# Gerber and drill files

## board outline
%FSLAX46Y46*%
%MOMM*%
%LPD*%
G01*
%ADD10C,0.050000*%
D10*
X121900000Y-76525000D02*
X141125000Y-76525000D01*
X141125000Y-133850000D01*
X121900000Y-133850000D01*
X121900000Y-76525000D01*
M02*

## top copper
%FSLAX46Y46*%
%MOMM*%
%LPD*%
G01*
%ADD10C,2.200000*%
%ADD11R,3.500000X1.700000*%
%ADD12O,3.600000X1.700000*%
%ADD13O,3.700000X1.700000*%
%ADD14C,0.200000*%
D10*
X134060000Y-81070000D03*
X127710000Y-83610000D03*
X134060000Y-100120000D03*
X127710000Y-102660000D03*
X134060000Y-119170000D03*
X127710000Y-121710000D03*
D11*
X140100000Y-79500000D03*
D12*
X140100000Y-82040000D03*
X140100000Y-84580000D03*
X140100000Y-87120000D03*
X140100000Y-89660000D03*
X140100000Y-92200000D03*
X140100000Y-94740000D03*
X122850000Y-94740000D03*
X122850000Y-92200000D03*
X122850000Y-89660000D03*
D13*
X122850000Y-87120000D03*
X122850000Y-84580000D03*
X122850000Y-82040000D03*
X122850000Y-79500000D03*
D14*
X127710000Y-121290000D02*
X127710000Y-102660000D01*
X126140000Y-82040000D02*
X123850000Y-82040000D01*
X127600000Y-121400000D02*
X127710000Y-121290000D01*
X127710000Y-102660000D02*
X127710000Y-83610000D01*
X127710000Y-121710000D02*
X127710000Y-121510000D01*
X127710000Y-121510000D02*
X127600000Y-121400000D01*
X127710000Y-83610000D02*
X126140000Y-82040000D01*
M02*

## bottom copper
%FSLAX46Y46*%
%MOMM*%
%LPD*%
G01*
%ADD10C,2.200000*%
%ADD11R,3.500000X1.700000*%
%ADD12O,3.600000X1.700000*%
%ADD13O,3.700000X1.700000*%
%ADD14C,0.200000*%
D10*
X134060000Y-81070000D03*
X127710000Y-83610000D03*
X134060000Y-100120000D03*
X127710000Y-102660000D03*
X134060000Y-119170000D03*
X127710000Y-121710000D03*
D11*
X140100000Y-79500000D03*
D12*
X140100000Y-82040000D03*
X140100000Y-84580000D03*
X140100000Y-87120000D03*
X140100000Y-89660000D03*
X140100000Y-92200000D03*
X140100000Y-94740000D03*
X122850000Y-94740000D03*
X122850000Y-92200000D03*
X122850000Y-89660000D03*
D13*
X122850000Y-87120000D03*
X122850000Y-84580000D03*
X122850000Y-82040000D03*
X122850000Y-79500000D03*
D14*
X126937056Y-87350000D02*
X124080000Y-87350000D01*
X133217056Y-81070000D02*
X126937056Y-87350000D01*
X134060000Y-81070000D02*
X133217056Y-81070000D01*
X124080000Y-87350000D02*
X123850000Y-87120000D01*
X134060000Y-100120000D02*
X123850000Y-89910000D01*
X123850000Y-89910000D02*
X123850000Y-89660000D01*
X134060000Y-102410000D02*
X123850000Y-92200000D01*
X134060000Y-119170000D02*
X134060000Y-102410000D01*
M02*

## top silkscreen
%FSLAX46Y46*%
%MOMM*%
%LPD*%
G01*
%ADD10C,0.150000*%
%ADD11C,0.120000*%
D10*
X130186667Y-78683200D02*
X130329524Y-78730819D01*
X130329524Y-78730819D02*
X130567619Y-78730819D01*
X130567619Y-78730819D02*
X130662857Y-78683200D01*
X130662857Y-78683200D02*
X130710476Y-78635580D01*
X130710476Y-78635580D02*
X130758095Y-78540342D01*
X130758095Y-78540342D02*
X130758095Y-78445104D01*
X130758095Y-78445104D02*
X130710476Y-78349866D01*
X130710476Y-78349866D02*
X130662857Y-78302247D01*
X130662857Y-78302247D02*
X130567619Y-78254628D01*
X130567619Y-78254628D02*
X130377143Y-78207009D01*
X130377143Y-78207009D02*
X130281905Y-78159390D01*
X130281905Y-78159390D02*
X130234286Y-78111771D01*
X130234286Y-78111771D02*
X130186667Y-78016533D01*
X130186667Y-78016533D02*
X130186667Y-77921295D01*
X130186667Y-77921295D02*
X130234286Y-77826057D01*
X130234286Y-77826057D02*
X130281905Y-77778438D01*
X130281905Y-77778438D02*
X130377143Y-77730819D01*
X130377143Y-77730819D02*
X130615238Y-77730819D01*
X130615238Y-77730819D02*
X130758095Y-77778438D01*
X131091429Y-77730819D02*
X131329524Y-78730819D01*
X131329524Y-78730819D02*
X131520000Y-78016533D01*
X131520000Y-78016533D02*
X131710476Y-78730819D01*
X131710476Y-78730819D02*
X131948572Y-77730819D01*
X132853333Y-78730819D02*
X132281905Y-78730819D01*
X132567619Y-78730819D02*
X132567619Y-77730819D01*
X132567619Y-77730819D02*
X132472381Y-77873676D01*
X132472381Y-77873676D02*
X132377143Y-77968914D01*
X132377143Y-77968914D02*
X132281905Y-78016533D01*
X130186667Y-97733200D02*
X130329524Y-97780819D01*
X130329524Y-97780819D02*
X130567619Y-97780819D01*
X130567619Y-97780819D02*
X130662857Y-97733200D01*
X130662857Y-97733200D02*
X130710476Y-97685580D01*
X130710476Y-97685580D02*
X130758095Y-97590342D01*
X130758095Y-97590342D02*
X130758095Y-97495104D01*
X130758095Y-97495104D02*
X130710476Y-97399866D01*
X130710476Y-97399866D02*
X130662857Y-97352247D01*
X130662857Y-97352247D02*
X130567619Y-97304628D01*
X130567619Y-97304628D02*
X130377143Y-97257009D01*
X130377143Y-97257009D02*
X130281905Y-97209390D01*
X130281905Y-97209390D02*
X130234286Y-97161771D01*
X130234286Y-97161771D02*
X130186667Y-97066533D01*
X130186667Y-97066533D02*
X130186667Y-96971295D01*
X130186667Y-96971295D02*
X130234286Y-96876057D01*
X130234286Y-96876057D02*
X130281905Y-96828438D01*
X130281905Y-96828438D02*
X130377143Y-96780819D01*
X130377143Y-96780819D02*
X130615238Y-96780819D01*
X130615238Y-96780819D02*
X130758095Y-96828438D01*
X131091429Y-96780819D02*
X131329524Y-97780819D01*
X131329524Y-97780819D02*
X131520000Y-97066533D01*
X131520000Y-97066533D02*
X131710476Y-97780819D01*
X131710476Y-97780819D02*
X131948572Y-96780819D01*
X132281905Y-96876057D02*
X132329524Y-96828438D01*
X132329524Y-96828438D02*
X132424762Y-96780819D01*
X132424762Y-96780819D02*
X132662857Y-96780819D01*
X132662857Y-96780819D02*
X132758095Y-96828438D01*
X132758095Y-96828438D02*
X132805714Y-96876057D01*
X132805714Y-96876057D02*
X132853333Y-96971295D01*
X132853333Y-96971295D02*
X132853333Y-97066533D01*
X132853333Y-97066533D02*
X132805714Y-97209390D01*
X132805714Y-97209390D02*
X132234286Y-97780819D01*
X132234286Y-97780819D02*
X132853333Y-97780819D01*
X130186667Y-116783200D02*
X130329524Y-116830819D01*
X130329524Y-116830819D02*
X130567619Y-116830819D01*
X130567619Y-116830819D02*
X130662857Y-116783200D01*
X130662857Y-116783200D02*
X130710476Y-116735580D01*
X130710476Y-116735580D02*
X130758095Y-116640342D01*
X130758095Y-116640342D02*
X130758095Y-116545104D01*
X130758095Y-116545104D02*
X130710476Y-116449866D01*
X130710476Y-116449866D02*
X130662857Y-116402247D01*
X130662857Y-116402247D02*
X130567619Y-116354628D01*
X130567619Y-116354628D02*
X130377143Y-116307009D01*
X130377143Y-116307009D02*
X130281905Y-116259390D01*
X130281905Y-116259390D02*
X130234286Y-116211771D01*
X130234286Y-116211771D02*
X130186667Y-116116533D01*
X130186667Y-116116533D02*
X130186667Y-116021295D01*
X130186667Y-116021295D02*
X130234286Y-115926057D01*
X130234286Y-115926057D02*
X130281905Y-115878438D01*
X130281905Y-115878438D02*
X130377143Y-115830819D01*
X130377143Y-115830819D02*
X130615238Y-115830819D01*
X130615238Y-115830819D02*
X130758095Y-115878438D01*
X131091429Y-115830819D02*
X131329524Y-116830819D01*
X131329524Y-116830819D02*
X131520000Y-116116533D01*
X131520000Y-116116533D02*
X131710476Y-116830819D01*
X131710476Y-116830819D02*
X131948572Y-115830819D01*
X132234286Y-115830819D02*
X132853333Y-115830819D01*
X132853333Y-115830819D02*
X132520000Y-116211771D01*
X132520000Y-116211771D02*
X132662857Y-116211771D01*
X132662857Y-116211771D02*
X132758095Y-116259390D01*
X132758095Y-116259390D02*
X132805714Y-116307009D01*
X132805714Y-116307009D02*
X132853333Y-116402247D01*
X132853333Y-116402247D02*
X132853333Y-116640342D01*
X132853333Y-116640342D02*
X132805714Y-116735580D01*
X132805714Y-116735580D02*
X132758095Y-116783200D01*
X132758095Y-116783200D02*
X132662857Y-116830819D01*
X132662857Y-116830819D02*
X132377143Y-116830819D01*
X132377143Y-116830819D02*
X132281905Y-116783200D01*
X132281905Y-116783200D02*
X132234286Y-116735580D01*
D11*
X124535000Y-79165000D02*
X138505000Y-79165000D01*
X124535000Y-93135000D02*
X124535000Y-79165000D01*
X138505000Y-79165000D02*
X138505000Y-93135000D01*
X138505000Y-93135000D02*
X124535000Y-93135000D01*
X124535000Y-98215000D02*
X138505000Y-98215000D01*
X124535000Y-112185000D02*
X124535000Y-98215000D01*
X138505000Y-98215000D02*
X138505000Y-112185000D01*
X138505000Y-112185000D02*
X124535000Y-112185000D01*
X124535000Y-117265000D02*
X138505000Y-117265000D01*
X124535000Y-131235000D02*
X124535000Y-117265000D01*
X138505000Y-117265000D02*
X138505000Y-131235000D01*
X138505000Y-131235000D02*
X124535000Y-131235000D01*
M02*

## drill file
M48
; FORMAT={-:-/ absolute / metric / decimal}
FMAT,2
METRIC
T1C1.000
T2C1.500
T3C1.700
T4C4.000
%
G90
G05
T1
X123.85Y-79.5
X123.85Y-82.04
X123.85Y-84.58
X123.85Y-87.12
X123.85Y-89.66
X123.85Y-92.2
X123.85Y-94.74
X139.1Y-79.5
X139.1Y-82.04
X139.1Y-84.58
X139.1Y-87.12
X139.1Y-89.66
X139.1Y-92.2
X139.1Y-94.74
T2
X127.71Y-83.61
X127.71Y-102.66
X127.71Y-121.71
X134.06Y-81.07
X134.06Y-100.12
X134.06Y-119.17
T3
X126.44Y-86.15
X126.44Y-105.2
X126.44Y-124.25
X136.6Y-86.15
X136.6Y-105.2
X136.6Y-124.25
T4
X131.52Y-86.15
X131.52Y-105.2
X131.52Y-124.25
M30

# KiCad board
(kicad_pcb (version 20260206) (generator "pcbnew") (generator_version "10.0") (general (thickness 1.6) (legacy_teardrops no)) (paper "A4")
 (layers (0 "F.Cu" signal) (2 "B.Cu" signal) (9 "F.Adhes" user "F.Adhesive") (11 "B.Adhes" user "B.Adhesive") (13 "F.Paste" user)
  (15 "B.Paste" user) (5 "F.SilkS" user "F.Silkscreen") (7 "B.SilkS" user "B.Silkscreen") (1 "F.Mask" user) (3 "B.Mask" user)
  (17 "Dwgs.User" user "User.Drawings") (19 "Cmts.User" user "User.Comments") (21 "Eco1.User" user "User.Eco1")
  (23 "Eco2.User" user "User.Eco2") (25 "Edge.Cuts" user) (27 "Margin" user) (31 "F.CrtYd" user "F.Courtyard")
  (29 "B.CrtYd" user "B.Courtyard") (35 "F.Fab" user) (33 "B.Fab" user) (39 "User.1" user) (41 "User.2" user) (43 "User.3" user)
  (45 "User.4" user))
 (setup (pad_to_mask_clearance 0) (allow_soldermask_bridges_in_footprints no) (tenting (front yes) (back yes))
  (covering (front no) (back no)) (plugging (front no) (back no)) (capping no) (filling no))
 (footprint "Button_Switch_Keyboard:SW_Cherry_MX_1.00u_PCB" (layer "F.Cu") (at 134.06 81.07)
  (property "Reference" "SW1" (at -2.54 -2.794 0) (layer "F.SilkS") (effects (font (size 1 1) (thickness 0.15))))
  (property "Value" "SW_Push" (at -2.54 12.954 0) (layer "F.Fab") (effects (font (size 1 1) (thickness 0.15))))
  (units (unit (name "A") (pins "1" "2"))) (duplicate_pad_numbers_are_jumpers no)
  (fp_line (start -9.525 -1.905) (end 4.445 -1.905) (stroke (width 0.12) (type solid)) (layer "F.SilkS"))
  (fp_line (start -9.525 12.065) (end -9.525 -1.905) (stroke (width 0.12) (type solid)) (layer "F.SilkS"))
  (fp_line (start 4.445 -1.905) (end 4.445 12.065) (stroke (width 0.12) (type solid)) (layer "F.SilkS"))
  (fp_line (start 4.445 12.065) (end -9.525 12.065) (stroke (width 0.12) (type solid)) (layer "F.SilkS"))
  (pad "" np_thru_hole circle (at -7.62 5.08) (size 1.7 1.7) (drill 1.7) (layers "*.Cu" "*.Mask"))
  (pad "" np_thru_hole circle (at -2.54 5.08) (size 4 4) (drill 4) (layers "*.Cu" "*.Mask"))
  (pad "" np_thru_hole circle (at 2.54 5.08) (size 1.7 1.7) (drill 1.7) (layers "*.Cu" "*.Mask"))
  (pad "1" thru_hole circle (at 0 0) (size 2.2 2.2) (drill 1.5) (layers "*.Cu" "*.Mask") (remove_unused_layers no)
   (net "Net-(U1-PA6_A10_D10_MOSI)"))
  (pad "2" thru_hole circle (at -6.35 2.54) (size 2.2 2.2) (drill 1.5) (layers "*.Cu" "*.Mask") (remove_unused_layers no) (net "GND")))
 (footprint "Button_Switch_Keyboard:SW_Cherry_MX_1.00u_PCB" (layer "F.Cu") (at 134.06 100.12)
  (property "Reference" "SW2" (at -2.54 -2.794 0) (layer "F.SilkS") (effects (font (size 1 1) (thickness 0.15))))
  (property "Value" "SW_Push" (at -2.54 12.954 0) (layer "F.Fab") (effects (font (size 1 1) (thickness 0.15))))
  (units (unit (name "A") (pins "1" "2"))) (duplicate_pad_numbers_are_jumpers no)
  (fp_line (start -9.525 -1.905) (end 4.445 -1.905) (stroke (width 0.12) (type solid)) (layer "F.SilkS"))
  (fp_line (start -9.525 12.065) (end -9.525 -1.905) (stroke (width 0.12) (type solid)) (layer "F.SilkS"))
  (fp_line (start 4.445 -1.905) (end 4.445 12.065) (stroke (width 0.12) (type solid)) (layer "F.SilkS"))
  (fp_line (start 4.445 12.065) (end -9.525 12.065) (stroke (width 0.12) (type solid)) (layer "F.SilkS"))
  (pad "" np_thru_hole circle (at -7.62 5.08) (size 1.7 1.7) (drill 1.7) (layers "*.Cu" "*.Mask"))
  (pad "" np_thru_hole circle (at -2.54 5.08) (size 4 4) (drill 4) (layers "*.Cu" "*.Mask"))
  (pad "" np_thru_hole circle (at 2.54 5.08) (size 1.7 1.7) (drill 1.7) (layers "*.Cu" "*.Mask"))
  (pad "1" thru_hole circle (at 0 0) (size 2.2 2.2) (drill 1.5) (layers "*.Cu" "*.Mask") (remove_unused_layers no)
   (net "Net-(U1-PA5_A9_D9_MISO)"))
  (pad "2" thru_hole circle (at -6.35 2.54) (size 2.2 2.2) (drill 1.5) (layers "*.Cu" "*.Mask") (remove_unused_layers no) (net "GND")))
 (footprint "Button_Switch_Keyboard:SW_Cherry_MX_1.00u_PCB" (layer "F.Cu") (at 134.06 119.17)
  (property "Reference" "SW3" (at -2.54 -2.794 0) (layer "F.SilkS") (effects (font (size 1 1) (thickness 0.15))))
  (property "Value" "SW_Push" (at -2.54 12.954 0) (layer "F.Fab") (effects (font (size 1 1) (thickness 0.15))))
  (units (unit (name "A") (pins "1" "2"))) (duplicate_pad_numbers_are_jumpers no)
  (fp_line (start -9.525 -1.905) (end 4.445 -1.905) (stroke (width 0.12) (type solid)) (layer "F.SilkS"))
  (fp_line (start -9.525 12.065) (end -9.525 -1.905) (stroke (width 0.12) (type solid)) (layer "F.SilkS"))
  (fp_line (start 4.445 -1.905) (end 4.445 12.065) (stroke (width 0.12) (type solid)) (layer "F.SilkS"))
  (fp_line (start 4.445 12.065) (end -9.525 12.065) (stroke (width 0.12) (type solid)) (layer "F.SilkS"))
  (pad "" np_thru_hole circle (at -7.62 5.08) (size 1.7 1.7) (drill 1.7) (layers "*.Cu" "*.Mask"))
  (pad "" np_thru_hole circle (at -2.54 5.08) (size 4 4) (drill 4) (layers "*.Cu" "*.Mask"))
  (pad "" np_thru_hole circle (at 2.54 5.08) (size 1.7 1.7) (drill 1.7) (layers "*.Cu" "*.Mask"))
  (pad "1" thru_hole circle (at 0 0) (size 2.2 2.2) (drill 1.5) (layers "*.Cu" "*.Mask") (remove_unused_layers no)
   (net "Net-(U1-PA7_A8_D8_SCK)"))
  (pad "2" thru_hole circle (at -6.35 2.54) (size 2.2 2.2) (drill 1.5) (layers "*.Cu" "*.Mask") (remove_unused_layers no) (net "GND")))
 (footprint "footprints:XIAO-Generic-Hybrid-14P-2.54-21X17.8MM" (layer "B.Cu") (at 131.475 87.12 180)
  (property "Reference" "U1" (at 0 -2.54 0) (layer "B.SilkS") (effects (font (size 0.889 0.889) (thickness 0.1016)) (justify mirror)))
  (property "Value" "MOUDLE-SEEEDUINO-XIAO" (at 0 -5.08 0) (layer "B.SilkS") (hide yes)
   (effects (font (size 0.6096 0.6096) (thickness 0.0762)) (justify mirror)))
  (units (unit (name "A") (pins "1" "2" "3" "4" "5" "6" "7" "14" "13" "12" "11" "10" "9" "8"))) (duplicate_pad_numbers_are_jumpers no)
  (pad "1" thru_hole rect (at -7.625 7.62 180) (size 3.5 1.7) (drill 1 (offset -1 0)) (layers "*.Cu" "*.Mask") (remove_unused_layers no)
   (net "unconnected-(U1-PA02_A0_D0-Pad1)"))
  (pad "2" thru_hole oval (at -7.625 5.08 180) (size 3.6 1.7) (drill 1 (offset -1 0)) (layers "*.Cu" "*.Mask") (remove_unused_layers no)
   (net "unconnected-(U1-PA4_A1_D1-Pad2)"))
  (pad "3" thru_hole oval (at -7.625 2.54 180) (size 3.6 1.7) (drill 1 (offset -1 0)) (layers "*.Cu" "*.Mask") (remove_unused_layers no)
   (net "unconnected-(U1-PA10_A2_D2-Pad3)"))
  (pad "4" thru_hole oval (at -7.625 0 180) (size 3.6 1.7) (drill 1 (offset -1 0)) (layers "*.Cu" "*.Mask") (remove_unused_layers no)
   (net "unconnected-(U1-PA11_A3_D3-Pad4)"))
  (pad "5" thru_hole oval (at -7.625 -2.54 180) (size 3.6 1.7) (drill 1 (offset -1 0)) (layers "*.Cu" "*.Mask") (remove_unused_layers no)
   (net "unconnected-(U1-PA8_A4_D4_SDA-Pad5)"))
  (pad "6" thru_hole oval (at -7.625 -5.08) (size 3.6 1.7) (drill 1 (offset 1 0)) (layers "*.Cu" "*.Mask") (remove_unused_layers no)
   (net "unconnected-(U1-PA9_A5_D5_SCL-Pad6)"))
  (pad "7" thru_hole oval (at -7.625 -7.62 180) (size 3.6 1.7) (drill 1 (offset -1 0)) (layers "*.Cu" "*.Mask") (remove_unused_layers no)
   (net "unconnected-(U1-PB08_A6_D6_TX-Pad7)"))
  (pad "8" thru_hole oval (at 7.625 -7.62 180) (size 3.6 1.7) (drill 1 (offset 1 0)) (layers "*.Cu" "*.Mask") (remove_unused_layers no)
   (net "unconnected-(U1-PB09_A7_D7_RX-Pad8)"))
  (pad "9" thru_hole oval (at 7.625 -5.08 180) (size 3.6 1.7) (drill 1 (offset 1 0)) (layers "*.Cu" "*.Mask") (remove_unused_layers no)
   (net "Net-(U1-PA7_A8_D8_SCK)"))
  (pad "10" thru_hole oval (at 7.625 -2.54 180) (size 3.6 1.7) (drill 1 (offset 1 0)) (layers "*.Cu" "*.Mask") (remove_unused_layers no)
   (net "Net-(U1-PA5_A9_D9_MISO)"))
  (pad "11" thru_hole oval (at 7.625 0 180) (size 3.7 1.7) (drill 1 (offset 1 0)) (layers "*.Cu" "*.Mask") (remove_unused_layers no)
   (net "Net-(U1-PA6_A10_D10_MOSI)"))
  (pad "12" thru_hole oval (at 7.625 2.54 180) (size 3.7 1.7) (drill 1 (offset 1 0)) (layers "*.Cu" "*.Mask") (remove_unused_layers no)
   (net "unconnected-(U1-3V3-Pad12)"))
  (pad "13" thru_hole oval (at 7.625 5.08 180) (size 3.7 1.7) (drill 1 (offset 1 0)) (layers "*.Cu" "*.Mask") (remove_unused_layers no)
   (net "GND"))
  (pad "14" thru_hole oval (at 7.625 7.62 180) (size 3.7 1.7) (drill 1 (offset 1 0)) (layers "*.Cu" "*.Mask") (remove_unused_layers no)
   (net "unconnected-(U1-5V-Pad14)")))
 (gr_rect (start 121.9 76.525) (end 141.125 133.85) (stroke (width 0.05) (type default)) (fill no) (layer "Edge.Cuts"))
 (segment (start 126.937056 87.35) (end 124.08 87.35) (width 0.2) (layer "B.Cu") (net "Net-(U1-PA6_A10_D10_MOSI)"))
 (segment (start 133.217056 81.07) (end 126.937056 87.35) (width 0.2) (layer "B.Cu") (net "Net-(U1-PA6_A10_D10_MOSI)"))
 (segment (start 134.06 81.07) (end 133.217056 81.07) (width 0.2) (layer "B.Cu") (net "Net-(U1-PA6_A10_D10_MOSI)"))
 (segment (start 124.08 87.35) (end 123.85 87.12) (width 0.2) (layer "B.Cu") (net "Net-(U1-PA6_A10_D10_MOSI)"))
 (segment (start 127.71 121.29) (end 127.71 102.66) (width 0.2) (layer "F.Cu") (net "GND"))
 (segment (start 126.14 82.04) (end 123.85 82.04) (width 0.2) (layer "F.Cu") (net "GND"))
 (segment (start 127.6 121.4) (end 127.71 121.29) (width 0.2) (layer "F.Cu") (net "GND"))
 (segment (start 127.71 102.66) (end 127.71 83.61) (width 0.2) (layer "F.Cu") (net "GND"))
 (segment (start 127.71 121.71) (end 127.71 121.51) (width 0.2) (layer "F.Cu") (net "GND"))
 (segment (start 127.71 121.51) (end 127.6 121.4) (width 0.2) (layer "F.Cu") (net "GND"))
 (segment (start 127.71 83.61) (end 126.14 82.04) (width 0.2) (layer "F.Cu") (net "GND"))
 (segment (start 134.06 100.12) (end 123.85 89.91) (width 0.2) (layer "B.Cu") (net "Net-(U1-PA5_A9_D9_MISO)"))
 (segment (start 123.85 89.91) (end 123.85 89.66) (width 0.2) (layer "B.Cu") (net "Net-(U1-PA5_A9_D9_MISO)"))
 (segment (start 134.06 102.41) (end 123.85 92.2) (width 0.2) (layer "B.Cu") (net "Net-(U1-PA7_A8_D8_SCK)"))
 (segment (start 134.06 119.17) (end 134.06 102.41) (width 0.2) (layer "B.Cu") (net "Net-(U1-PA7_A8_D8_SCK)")))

